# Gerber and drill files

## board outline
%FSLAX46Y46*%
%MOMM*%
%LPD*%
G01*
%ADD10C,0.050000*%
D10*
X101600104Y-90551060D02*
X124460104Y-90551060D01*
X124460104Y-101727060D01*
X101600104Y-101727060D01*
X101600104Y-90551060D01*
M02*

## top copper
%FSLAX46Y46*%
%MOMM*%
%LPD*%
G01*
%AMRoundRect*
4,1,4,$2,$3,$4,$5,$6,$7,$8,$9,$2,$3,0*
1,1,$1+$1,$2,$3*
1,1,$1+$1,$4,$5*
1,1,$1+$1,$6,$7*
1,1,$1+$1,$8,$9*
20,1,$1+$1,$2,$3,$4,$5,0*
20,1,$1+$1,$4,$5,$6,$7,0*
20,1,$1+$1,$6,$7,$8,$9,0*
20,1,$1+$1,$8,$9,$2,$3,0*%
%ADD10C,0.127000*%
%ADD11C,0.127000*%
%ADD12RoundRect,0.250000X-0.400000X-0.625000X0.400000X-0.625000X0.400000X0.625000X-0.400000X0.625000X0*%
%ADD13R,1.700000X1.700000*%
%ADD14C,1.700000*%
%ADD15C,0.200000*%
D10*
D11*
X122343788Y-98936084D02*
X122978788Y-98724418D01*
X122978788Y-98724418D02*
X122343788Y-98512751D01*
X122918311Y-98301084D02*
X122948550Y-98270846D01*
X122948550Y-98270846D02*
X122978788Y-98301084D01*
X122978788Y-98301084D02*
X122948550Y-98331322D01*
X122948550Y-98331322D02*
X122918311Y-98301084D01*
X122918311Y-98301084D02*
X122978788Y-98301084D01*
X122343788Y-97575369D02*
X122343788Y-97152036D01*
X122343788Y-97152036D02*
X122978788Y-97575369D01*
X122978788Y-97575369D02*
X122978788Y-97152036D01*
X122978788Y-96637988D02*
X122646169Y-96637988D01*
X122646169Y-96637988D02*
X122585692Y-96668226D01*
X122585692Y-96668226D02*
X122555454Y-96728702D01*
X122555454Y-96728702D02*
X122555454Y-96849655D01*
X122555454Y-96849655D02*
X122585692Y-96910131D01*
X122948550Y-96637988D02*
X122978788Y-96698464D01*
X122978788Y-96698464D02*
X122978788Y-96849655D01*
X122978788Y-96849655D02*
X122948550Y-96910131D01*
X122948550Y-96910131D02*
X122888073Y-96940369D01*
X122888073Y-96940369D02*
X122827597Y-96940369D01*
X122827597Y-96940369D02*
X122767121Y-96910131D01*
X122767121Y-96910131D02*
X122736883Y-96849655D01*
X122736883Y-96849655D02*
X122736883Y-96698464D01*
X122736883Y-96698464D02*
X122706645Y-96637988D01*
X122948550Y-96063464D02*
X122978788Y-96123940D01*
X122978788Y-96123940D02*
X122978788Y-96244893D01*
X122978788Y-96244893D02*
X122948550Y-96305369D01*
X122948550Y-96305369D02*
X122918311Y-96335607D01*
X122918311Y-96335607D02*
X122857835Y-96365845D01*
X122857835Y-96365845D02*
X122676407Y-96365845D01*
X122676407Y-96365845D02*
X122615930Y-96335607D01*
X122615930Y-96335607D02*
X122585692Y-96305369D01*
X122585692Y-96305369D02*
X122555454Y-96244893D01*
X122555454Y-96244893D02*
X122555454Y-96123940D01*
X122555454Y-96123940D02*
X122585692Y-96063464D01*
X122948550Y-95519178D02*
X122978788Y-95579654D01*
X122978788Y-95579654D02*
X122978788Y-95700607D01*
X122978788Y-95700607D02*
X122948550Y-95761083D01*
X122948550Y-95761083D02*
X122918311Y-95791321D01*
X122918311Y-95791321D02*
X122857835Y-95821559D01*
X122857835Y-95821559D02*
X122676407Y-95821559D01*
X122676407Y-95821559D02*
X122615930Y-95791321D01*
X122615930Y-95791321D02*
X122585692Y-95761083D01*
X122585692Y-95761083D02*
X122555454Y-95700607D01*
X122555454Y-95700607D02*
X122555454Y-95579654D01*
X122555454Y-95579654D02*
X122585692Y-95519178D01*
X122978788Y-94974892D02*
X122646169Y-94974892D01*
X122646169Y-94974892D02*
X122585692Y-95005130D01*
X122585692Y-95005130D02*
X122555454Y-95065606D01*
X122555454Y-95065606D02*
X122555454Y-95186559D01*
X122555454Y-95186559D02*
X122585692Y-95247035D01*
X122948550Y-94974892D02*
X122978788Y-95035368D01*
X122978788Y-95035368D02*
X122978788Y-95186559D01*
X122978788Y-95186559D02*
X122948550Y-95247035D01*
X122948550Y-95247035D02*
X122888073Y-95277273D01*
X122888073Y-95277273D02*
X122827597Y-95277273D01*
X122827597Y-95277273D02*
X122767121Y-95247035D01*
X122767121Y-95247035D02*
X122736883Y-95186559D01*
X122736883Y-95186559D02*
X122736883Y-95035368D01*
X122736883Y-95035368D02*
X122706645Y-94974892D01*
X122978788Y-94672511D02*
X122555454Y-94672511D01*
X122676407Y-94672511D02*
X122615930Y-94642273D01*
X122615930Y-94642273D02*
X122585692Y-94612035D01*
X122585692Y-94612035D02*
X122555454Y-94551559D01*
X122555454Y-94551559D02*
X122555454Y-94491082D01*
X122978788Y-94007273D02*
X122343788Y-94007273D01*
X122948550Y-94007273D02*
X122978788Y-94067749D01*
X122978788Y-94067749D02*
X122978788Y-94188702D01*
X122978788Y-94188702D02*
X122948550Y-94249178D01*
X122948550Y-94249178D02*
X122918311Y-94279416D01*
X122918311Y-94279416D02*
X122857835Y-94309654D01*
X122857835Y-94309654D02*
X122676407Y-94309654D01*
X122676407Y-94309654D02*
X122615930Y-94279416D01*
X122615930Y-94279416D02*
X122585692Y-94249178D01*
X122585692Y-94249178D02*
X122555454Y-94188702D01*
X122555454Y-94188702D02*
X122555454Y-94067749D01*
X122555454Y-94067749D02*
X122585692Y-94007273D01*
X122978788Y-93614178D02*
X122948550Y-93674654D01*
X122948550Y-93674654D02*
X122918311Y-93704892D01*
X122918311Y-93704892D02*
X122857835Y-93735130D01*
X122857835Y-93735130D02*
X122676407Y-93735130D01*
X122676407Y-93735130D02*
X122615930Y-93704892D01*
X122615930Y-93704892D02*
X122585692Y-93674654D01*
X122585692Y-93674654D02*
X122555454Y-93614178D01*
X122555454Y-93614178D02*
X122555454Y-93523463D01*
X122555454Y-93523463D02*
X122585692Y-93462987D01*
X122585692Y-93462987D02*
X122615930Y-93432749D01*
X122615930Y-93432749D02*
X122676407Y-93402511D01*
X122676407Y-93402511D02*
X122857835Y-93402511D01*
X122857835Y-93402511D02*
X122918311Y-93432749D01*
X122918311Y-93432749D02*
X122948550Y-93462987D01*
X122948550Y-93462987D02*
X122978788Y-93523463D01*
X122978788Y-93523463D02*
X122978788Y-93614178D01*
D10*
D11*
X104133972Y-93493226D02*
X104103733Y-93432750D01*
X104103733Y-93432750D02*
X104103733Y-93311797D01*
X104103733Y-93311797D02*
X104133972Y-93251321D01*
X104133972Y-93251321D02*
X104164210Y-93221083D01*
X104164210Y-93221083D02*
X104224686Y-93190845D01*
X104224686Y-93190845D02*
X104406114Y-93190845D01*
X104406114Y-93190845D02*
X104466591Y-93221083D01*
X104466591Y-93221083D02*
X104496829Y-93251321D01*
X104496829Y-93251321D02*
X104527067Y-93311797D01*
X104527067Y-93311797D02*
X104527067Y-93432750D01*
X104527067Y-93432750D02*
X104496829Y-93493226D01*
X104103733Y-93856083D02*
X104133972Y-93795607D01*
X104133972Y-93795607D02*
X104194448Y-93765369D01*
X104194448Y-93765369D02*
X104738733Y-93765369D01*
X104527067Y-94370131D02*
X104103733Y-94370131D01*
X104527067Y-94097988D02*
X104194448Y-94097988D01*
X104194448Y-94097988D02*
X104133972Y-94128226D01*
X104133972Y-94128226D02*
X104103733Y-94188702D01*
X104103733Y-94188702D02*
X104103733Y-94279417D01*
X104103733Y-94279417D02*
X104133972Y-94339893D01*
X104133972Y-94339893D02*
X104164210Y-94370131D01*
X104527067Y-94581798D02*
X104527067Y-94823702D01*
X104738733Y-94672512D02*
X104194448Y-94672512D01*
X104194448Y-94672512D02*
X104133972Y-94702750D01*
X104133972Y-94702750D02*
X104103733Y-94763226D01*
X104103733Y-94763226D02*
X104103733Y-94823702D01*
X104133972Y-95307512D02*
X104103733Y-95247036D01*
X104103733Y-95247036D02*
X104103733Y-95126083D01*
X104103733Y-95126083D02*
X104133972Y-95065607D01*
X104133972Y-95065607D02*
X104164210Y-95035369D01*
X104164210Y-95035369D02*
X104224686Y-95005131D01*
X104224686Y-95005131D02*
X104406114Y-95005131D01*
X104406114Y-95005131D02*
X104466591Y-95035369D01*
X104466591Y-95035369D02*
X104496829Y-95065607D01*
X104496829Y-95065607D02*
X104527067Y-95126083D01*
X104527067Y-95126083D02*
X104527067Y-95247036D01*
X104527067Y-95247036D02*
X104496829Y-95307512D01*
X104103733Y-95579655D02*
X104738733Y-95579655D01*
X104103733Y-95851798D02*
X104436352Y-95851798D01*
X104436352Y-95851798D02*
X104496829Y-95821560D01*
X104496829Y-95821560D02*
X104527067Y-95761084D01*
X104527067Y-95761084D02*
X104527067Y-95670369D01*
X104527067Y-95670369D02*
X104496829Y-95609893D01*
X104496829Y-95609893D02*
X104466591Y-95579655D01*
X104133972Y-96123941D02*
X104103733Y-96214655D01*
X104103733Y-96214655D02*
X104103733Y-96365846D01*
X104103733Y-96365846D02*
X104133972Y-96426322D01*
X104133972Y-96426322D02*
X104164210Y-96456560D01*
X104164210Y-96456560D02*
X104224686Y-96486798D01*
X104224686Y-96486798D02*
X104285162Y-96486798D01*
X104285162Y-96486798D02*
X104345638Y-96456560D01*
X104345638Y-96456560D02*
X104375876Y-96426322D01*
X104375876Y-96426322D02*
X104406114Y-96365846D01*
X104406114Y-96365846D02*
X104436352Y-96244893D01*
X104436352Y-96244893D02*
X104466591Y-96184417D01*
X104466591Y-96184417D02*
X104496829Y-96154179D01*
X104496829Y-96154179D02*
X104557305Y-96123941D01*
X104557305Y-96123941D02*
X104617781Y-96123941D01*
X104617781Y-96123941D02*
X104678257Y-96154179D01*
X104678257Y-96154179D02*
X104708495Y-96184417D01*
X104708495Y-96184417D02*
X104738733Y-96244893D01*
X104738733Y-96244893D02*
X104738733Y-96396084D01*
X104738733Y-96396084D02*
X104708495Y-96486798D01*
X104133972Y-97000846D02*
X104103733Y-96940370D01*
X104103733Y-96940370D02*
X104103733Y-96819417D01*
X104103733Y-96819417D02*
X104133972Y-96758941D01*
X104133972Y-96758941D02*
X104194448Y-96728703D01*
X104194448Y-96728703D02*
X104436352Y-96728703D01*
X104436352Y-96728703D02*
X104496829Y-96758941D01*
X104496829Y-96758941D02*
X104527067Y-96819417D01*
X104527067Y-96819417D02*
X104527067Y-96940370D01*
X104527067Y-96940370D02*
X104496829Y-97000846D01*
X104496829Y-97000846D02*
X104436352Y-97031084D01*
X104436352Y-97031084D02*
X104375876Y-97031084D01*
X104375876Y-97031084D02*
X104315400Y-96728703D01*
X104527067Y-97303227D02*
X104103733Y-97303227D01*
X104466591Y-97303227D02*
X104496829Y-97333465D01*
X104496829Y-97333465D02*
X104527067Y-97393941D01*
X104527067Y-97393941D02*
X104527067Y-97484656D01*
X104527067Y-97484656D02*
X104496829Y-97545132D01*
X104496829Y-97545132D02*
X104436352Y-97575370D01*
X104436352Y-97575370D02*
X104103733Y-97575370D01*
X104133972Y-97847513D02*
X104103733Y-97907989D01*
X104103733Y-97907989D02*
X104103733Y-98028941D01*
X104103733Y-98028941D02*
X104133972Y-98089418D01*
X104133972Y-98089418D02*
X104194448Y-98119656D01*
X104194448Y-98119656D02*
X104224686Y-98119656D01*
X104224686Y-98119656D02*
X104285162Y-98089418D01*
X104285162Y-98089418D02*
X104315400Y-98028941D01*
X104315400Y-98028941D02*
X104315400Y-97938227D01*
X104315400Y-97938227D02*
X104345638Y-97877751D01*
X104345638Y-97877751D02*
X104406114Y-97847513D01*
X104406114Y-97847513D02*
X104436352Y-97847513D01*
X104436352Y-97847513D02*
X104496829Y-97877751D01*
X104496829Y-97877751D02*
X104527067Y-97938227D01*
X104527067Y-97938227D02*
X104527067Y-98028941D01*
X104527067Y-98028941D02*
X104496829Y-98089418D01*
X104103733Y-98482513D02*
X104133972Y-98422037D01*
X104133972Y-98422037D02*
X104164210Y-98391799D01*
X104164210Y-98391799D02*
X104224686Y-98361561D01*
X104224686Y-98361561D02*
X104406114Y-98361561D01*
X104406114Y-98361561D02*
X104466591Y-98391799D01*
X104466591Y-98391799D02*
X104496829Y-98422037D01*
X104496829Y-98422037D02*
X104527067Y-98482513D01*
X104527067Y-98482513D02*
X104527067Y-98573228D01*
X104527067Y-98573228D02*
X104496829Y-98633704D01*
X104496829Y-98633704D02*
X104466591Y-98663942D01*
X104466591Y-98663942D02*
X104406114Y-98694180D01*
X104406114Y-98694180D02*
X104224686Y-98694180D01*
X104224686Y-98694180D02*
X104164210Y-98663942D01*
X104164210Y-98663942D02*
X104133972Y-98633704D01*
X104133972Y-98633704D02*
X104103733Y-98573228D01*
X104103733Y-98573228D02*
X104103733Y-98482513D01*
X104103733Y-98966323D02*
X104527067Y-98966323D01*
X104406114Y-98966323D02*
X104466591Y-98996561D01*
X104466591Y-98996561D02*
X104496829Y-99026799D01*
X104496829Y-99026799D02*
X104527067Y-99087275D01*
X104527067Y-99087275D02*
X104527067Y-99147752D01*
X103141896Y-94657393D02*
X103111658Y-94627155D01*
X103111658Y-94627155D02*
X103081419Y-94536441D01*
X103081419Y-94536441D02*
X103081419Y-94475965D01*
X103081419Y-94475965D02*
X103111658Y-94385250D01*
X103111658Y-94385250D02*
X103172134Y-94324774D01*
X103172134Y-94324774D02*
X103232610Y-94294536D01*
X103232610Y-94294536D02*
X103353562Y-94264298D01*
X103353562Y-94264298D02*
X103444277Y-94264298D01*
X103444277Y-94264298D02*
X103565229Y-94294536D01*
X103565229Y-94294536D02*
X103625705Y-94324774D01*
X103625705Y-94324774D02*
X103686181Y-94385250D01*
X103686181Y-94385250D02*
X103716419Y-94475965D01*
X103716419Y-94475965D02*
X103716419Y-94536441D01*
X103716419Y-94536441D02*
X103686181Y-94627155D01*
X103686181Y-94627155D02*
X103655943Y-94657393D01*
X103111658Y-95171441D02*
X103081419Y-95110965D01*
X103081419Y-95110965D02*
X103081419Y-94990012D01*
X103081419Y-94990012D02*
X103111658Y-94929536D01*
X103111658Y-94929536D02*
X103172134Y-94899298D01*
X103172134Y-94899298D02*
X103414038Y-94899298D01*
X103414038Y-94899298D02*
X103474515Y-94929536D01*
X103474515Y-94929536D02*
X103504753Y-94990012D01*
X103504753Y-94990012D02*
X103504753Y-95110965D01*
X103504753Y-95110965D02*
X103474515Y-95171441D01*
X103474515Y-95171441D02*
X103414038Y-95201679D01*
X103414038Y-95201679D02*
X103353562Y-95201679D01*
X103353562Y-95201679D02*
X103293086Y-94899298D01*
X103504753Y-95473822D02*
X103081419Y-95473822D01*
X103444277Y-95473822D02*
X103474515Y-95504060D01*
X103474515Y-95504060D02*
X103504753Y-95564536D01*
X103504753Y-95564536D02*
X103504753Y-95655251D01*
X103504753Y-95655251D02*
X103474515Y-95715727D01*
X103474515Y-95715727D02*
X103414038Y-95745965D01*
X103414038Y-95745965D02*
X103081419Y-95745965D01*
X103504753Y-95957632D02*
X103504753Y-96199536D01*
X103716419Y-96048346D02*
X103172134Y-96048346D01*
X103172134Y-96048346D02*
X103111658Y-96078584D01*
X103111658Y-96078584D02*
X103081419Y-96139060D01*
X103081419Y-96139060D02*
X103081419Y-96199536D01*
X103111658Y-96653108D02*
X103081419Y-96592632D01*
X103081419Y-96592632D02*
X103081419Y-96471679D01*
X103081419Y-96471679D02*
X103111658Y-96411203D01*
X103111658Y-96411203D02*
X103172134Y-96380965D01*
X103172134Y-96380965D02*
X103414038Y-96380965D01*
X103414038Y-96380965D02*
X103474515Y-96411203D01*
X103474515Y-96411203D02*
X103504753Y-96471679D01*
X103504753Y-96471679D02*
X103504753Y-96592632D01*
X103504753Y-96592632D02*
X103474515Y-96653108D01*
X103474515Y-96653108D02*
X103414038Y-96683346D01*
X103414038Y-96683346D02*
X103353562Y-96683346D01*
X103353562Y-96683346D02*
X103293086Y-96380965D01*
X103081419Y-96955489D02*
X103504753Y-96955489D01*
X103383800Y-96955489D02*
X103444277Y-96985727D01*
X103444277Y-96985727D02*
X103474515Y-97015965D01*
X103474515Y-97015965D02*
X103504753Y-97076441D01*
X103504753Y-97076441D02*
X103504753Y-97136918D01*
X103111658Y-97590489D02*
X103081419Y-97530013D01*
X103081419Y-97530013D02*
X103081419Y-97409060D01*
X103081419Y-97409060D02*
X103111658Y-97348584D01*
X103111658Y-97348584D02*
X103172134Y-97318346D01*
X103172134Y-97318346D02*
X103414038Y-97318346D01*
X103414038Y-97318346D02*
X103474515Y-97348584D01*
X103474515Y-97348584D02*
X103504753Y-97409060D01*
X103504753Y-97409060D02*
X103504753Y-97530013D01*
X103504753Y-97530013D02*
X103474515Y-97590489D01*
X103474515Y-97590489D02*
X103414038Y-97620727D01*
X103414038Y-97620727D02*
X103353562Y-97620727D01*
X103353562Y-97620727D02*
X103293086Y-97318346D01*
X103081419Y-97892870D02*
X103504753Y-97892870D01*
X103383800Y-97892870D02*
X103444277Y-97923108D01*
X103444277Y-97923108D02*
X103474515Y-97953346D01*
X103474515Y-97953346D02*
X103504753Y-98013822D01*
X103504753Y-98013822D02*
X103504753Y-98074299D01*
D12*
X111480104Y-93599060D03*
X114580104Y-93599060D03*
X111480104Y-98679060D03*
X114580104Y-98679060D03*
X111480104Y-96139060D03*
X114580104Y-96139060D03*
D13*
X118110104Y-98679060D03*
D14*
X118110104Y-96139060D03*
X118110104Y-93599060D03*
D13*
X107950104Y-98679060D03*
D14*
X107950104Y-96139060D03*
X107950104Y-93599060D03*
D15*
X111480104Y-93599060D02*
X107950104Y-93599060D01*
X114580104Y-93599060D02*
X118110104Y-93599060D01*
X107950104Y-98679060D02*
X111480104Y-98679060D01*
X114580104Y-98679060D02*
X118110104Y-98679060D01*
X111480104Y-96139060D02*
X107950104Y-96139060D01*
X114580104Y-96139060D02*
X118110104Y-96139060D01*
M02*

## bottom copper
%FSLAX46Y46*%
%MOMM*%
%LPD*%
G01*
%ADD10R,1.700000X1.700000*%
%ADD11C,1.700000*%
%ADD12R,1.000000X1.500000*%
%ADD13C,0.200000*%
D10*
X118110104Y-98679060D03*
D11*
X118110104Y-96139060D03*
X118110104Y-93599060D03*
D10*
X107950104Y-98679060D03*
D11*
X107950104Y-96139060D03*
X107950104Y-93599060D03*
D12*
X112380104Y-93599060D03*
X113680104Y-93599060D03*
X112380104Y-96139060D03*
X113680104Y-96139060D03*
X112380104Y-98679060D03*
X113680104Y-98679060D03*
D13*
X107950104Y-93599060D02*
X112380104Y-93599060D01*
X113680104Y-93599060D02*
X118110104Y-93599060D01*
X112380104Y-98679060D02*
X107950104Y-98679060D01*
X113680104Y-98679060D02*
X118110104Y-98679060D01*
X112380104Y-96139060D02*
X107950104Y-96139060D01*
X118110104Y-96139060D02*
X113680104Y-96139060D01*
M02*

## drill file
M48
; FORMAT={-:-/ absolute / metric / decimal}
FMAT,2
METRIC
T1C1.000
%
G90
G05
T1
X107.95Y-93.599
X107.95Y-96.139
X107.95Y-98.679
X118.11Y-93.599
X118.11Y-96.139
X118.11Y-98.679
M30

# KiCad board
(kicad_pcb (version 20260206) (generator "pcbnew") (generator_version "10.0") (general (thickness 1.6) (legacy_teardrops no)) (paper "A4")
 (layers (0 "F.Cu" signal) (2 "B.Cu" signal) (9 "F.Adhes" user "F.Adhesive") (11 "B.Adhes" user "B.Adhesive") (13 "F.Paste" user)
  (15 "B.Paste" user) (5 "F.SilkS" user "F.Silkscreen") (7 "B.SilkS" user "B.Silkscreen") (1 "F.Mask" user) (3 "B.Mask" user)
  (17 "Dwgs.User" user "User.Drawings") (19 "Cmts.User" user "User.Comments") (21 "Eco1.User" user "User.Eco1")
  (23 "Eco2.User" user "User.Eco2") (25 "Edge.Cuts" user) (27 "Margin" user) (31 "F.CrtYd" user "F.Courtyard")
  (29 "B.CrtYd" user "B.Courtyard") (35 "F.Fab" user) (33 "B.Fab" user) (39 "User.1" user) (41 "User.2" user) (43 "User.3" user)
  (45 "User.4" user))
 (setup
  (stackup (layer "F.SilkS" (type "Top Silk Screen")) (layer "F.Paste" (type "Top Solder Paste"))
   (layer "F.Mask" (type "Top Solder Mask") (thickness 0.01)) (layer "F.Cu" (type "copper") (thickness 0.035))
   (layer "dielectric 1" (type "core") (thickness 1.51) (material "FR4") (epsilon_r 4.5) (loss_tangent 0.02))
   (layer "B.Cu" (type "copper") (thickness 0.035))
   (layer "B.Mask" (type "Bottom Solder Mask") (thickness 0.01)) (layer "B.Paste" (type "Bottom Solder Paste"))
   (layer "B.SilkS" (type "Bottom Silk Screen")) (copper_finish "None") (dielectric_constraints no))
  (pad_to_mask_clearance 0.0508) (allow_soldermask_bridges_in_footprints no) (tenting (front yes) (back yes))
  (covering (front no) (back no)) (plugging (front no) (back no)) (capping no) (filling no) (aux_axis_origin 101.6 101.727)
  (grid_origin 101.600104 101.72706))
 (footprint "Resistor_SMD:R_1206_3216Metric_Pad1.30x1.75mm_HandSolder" (layer "F.Cu") (at 113.030104 93.59906)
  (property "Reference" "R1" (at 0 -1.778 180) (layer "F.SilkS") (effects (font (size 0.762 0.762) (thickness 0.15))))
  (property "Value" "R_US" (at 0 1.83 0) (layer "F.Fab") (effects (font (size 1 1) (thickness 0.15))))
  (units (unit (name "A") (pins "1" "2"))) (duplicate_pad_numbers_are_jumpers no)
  (pad "1" smd roundrect (at -1.55 0) (size 1.3 1.75) (layers "F.Cu" "F.Mask" "F.Paste") (roundrect_rratio 0.192308) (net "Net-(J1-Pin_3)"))
  (pad "2" smd roundrect (at 1.55 0) (size 1.3 1.75) (layers "F.Cu" "F.Mask" "F.Paste") (roundrect_rratio 0.192308) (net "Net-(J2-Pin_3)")))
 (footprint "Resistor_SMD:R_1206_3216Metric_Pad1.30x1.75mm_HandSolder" (layer "F.Cu") (at 113.030104 98.67906)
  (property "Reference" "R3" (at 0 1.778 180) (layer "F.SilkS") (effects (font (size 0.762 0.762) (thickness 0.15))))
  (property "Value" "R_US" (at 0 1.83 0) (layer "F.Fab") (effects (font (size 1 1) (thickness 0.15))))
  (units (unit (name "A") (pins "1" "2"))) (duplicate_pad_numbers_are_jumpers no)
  (pad "1" smd roundrect (at -1.55 0) (size 1.3 1.75) (layers "F.Cu" "F.Mask" "F.Paste") (roundrect_rratio 0.192308) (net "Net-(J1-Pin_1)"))
  (pad "2" smd roundrect (at 1.55 0) (size 1.3 1.75) (layers "F.Cu" "F.Mask" "F.Paste") (roundrect_rratio 0.192308) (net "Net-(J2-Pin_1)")))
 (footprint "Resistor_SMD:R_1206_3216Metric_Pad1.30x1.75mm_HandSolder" (layer "F.Cu") (at 113.030104 96.13906)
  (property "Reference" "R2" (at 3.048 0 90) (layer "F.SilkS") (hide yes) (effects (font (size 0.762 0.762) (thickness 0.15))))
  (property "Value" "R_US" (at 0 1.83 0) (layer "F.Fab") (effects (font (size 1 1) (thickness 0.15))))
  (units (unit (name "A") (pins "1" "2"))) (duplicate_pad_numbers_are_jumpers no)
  (pad "1" smd roundrect (at -1.55 0) (size 1.3 1.75) (layers "F.Cu" "F.Mask" "F.Paste") (roundrect_rratio 0.192308) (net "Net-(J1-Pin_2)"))
  (pad "2" smd roundrect (at 1.55 0) (size 1.3 1.75) (layers "F.Cu" "F.Mask" "F.Paste") (roundrect_rratio 0.192308) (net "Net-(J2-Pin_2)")))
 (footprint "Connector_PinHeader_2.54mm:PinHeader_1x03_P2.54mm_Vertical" (layer "F.Cu") (at 118.110104 98.67906 180)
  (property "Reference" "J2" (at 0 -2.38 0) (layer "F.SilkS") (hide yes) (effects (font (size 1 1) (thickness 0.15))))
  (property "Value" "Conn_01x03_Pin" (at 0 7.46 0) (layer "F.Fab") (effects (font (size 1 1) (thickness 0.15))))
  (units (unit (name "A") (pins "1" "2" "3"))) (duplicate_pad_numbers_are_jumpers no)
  (pad "1" thru_hole rect (at 0 0 180) (size 1.7 1.7) (drill 1) (layers "*.Cu" "*.Mask") (remove_unused_layers no) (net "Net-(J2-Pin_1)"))
  (pad "2" thru_hole circle (at 0 2.54 180) (size 1.7 1.7) (drill 1) (layers "*.Cu" "*.Mask") (remove_unused_layers no)
   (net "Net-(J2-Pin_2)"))
  (pad "3" thru_hole circle (at 0 5.08 180) (size 1.7 1.7) (drill 1) (layers "*.Cu" "*.Mask") (remove_unused_layers no)
   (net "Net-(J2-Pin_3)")))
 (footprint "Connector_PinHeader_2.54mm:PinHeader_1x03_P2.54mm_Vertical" (layer "F.Cu") (at 107.950104 98.67906 180)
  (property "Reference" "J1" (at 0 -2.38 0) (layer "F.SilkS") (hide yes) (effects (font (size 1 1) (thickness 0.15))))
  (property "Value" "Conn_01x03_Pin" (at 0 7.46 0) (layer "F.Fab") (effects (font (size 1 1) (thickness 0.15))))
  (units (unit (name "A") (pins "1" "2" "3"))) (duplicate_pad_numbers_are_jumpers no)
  (pad "1" thru_hole rect (at 0 0 180) (size 1.7 1.7) (drill 1) (layers "*.Cu" "*.Mask") (remove_unused_layers no) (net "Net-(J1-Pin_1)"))
  (pad "2" thru_hole circle (at 0 2.54 180) (size 1.7 1.7) (drill 1) (layers "*.Cu" "*.Mask") (remove_unused_layers no)
   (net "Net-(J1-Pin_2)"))
  (pad "3" thru_hole circle (at 0 5.08 180) (size 1.7 1.7) (drill 1) (layers "*.Cu" "*.Mask") (remove_unused_layers no)
   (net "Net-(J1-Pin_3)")))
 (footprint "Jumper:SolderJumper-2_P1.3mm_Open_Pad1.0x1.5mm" (layer "B.Cu") (at 113.030104 93.59906)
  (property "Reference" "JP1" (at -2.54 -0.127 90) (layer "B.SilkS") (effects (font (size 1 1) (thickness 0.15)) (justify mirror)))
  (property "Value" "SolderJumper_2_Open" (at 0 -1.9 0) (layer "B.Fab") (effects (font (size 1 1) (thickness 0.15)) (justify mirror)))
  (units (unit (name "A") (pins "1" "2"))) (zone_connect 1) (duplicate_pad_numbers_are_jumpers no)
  (pad "1" smd rect (at -0.65 0) (size 1 1.5) (layers "B.Cu" "B.Mask") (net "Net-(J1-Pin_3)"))
  (pad "2" smd rect (at 0.65 0) (size 1 1.5) (layers "B.Cu" "B.Mask") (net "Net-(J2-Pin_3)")))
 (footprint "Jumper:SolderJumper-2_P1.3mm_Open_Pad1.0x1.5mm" (layer "B.Cu") (at 113.030104 96.13906)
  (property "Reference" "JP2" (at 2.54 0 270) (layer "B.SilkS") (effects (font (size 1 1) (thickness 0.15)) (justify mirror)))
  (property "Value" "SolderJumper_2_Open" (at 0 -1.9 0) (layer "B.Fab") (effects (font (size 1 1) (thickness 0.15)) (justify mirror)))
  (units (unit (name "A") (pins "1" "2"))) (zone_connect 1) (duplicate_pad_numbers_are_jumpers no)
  (pad "1" smd rect (at -0.65 0) (size 1 1.5) (layers "B.Cu" "B.Mask") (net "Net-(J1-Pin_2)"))
  (pad "2" smd rect (at 0.65 0) (size 1 1.5) (layers "B.Cu" "B.Mask") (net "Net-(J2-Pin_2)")))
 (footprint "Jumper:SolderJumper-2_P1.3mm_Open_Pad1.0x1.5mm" (layer "B.Cu") (at 113.030104 98.67906)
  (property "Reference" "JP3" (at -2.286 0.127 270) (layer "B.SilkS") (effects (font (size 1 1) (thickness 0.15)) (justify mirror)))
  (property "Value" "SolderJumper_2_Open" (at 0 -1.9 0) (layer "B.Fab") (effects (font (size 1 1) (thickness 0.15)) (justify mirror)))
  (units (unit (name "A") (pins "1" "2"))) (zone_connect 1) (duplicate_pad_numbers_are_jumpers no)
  (pad "1" smd rect (at -0.65 0) (size 1 1.5) (layers "B.Cu" "B.Mask") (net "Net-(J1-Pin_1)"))
  (pad "2" smd rect (at 0.65 0) (size 1 1.5) (layers "B.Cu" "B.Mask") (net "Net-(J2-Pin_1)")))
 (gr_rect (start 101.600104 90.55106) (end 124.460104 101.72706) (stroke (width 0.05) (type solid)) (fill no) (layer "Edge.Cuts"))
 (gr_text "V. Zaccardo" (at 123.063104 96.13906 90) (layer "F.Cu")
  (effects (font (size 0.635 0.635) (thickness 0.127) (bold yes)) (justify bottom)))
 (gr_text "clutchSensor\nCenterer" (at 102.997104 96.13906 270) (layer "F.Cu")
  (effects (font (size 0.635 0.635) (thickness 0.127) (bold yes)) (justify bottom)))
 (segment (start 111.480104 93.59906) (end 107.950104 93.59906) (width 0.2) (layer "F.Cu") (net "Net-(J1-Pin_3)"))
 (segment (start 107.950104 93.59906) (end 112.380104 93.59906) (width 0.2) (layer "B.Cu") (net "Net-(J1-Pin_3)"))
 (segment (start 114.580104 93.59906) (end 118.110104 93.59906) (width 0.2) (layer "F.Cu") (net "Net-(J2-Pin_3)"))
 (segment (start 113.680104 93.59906) (end 118.110104 93.59906) (width 0.2) (layer "B.Cu") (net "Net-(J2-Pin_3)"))
 (segment (start 107.950104 98.67906) (end 111.480104 98.67906) (width 0.2) (layer "F.Cu") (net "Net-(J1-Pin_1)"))
 (segment (start 112.380104 98.67906) (end 107.950104 98.67906) (width 0.2) (layer "B.Cu") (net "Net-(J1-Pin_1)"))
 (segment (start 114.580104 98.67906) (end 118.110104 98.67906) (width 0.2) (layer "F.Cu") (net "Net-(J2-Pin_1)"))
 (segment (start 113.680104 98.67906) (end 118.110104 98.67906) (width 0.2) (layer "B.Cu") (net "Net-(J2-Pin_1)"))
 (segment (start 111.480104 96.13906) (end 107.950104 96.13906) (width 0.2) (layer "F.Cu") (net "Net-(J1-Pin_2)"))
 (segment (start 112.380104 96.13906) (end 107.950104 96.13906) (width 0.2) (layer "B.Cu") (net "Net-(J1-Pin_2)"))
 (segment (start 114.580104 96.13906) (end 118.110104 96.13906) (width 0.2) (layer "F.Cu") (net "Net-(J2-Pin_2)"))
 (segment (start 118.110104 96.13906) (end 113.680104 96.13906) (width 0.2) (layer "B.Cu") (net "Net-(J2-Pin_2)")))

